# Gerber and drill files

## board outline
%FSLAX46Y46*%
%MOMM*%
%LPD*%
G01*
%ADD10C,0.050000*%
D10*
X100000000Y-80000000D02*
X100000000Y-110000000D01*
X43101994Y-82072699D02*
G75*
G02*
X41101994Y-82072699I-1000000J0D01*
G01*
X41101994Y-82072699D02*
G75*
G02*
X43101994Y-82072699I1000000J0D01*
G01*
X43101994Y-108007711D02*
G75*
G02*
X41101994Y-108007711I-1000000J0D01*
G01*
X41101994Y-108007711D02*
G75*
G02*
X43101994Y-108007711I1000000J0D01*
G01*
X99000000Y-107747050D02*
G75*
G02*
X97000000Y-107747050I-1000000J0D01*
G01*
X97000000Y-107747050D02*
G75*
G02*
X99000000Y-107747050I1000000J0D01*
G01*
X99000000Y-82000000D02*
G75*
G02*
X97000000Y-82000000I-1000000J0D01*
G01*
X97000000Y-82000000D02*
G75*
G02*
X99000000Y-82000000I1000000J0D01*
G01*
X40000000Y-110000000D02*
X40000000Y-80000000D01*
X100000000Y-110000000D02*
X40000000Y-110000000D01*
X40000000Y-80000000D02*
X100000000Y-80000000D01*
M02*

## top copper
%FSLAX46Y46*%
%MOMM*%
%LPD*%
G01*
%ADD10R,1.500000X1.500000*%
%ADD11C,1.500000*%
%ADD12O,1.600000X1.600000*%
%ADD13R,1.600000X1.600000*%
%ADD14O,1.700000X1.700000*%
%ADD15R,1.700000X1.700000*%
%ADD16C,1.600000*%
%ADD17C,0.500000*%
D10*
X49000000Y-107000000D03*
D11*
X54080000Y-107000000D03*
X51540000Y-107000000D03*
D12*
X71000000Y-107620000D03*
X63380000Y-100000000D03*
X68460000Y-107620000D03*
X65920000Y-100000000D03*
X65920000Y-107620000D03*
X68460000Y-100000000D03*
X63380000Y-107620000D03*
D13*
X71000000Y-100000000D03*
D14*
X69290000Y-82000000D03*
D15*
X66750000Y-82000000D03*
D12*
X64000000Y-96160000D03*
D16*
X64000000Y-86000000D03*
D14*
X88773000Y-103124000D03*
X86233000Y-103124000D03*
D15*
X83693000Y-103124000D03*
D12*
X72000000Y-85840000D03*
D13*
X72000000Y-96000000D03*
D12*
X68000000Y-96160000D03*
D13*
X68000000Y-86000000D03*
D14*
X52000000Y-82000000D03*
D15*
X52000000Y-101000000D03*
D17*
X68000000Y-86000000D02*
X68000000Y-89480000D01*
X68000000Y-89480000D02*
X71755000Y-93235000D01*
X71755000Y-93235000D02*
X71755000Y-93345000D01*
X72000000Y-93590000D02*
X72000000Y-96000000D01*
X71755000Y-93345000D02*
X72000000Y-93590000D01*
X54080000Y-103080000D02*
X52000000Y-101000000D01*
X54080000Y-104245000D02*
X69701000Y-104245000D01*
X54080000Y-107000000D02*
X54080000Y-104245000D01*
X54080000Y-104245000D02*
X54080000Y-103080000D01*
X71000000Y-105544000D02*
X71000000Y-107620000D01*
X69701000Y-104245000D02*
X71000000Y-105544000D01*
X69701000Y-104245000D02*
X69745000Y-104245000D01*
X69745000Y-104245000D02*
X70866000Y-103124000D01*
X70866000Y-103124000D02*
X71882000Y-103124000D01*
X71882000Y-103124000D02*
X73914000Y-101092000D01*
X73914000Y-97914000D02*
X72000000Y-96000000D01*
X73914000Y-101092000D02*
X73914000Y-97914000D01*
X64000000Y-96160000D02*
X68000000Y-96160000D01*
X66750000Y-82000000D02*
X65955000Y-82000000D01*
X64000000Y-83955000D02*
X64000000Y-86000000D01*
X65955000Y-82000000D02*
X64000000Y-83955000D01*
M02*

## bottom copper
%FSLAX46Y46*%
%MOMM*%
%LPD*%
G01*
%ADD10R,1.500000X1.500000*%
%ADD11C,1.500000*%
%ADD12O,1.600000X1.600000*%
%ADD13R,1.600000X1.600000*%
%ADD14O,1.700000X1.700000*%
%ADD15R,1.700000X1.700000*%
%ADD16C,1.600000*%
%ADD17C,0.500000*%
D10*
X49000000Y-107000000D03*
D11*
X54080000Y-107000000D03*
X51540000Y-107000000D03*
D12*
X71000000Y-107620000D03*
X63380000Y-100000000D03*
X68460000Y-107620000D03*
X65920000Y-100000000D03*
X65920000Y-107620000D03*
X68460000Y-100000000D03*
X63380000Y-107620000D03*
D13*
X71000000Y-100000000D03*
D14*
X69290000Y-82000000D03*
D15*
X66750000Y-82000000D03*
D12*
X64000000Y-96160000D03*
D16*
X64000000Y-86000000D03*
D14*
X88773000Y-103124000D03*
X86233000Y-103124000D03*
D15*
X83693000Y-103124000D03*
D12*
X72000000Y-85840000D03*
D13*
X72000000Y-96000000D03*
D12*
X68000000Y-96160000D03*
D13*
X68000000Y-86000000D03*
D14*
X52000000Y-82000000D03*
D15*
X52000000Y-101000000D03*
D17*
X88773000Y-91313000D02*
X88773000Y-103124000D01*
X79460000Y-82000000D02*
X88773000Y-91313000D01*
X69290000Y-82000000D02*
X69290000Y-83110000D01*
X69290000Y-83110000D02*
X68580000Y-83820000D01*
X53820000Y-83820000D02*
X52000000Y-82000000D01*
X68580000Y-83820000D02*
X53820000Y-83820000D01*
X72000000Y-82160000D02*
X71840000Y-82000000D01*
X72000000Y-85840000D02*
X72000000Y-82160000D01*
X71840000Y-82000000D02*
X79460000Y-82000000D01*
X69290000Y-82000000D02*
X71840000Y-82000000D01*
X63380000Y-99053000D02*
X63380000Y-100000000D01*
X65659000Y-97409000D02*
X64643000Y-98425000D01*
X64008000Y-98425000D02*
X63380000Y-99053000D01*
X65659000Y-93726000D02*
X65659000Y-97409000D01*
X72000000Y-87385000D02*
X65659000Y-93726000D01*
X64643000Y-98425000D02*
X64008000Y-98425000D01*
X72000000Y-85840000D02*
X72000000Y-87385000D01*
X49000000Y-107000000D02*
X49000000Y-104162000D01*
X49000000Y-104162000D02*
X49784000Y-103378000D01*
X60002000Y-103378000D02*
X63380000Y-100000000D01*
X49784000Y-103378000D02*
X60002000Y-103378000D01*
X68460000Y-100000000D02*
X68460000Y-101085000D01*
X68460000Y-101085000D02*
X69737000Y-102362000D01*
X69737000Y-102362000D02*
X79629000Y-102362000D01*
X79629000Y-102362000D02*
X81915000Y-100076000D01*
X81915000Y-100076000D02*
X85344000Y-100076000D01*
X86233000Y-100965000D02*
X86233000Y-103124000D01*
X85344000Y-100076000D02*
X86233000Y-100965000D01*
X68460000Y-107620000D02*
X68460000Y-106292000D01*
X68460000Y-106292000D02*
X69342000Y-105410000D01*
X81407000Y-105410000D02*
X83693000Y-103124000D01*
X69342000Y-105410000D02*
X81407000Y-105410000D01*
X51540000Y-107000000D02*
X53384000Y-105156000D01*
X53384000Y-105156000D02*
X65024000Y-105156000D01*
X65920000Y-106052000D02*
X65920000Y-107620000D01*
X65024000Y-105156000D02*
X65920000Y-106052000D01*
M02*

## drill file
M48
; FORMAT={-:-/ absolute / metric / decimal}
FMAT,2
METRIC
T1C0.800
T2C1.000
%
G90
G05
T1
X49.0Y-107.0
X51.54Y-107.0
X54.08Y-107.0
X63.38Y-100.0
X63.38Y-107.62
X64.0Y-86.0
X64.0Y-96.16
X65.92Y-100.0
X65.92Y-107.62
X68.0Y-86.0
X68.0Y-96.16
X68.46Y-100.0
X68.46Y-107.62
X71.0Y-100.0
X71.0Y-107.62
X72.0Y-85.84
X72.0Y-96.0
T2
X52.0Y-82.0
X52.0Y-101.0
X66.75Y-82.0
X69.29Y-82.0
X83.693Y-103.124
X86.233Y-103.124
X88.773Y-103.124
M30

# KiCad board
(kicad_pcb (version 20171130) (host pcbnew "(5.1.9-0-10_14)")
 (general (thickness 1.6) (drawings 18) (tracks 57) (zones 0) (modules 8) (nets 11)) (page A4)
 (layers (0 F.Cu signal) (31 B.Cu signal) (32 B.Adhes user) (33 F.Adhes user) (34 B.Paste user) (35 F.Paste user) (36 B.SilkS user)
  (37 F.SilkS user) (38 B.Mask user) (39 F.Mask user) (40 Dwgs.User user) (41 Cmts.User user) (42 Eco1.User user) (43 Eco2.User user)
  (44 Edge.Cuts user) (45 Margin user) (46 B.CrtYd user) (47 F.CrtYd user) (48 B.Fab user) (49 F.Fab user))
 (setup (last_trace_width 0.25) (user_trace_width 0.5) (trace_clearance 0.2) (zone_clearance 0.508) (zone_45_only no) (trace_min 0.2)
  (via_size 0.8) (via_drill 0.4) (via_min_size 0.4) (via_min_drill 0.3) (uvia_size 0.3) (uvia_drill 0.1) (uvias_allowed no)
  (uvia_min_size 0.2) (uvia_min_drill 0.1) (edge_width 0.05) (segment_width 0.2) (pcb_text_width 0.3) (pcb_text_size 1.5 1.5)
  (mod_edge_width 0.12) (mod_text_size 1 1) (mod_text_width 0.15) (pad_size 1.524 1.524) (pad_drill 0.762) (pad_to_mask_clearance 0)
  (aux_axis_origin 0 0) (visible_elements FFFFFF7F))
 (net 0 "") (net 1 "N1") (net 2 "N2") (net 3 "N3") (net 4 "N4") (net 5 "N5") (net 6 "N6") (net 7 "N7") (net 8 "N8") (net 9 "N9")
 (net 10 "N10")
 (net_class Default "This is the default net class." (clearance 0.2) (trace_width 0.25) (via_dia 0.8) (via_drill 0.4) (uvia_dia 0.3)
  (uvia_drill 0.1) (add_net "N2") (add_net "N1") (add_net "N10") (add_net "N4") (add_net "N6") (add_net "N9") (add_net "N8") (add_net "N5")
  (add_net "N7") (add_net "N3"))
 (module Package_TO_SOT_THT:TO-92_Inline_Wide (layer F.Cu) (at 49 107)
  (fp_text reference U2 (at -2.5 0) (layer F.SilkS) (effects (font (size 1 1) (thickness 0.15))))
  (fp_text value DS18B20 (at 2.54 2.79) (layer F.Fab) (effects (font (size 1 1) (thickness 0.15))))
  (pad 1 thru_hole rect (at 0 0) (size 1.5 1.5) (drill 0.8) (layers *.Cu *.Mask) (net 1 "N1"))
  (pad 3 thru_hole circle (at 5.08 0) (size 1.5 1.5) (drill 0.8) (layers *.Cu *.Mask) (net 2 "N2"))
  (pad 2 thru_hole circle (at 2.54 0) (size 1.5 1.5) (drill 0.8) (layers *.Cu *.Mask) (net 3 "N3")))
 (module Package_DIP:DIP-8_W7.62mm (layer F.Cu) (at 71 100 270)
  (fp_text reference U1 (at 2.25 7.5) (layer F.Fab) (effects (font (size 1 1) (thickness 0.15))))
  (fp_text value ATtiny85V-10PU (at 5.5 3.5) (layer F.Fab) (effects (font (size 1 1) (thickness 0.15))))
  (pad 8 thru_hole oval (at 7.62 0 270) (size 1.6 1.6) (drill 0.8) (layers *.Cu *.Mask) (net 2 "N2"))
  (pad 4 thru_hole oval (at 0 7.62 270) (size 1.6 1.6) (drill 0.8) (layers *.Cu *.Mask) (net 1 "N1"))
  (pad 7 thru_hole oval (at 7.62 2.54 270) (size 1.6 1.6) (drill 0.8) (layers *.Cu *.Mask) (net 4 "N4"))
  (pad 3 thru_hole oval (at 0 5.08 270) (size 1.6 1.6) (drill 0.8) (layers *.Cu *.Mask) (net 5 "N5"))
  (pad 6 thru_hole oval (at 7.62 5.08 270) (size 1.6 1.6) (drill 0.8) (layers *.Cu *.Mask) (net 3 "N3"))
  (pad 2 thru_hole oval (at 0 2.54 270) (size 1.6 1.6) (drill 0.8) (layers *.Cu *.Mask) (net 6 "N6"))
  (pad 5 thru_hole oval (at 7.62 7.62 270) (size 1.6 1.6) (drill 0.8) (layers *.Cu *.Mask) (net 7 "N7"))
  (pad 1 thru_hole rect (at 0 0 270) (size 1.6 1.6) (drill 0.8) (layers *.Cu *.Mask) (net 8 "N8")))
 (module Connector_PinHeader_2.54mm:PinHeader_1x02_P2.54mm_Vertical (layer F.Cu) (at 66.75 82 90)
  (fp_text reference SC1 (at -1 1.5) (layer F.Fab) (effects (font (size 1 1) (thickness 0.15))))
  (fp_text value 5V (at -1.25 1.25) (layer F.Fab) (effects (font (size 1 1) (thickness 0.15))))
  (pad 2 thru_hole oval (at 0 2.54 90) (size 1.7 1.7) (drill 1) (layers *.Cu *.Mask) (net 1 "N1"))
  (pad 1 thru_hole rect (at 0 0 90) (size 1.7 1.7) (drill 1) (layers *.Cu *.Mask) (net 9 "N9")))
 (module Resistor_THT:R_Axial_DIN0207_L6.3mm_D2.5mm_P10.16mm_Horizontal (layer F.Cu) (at 64 86 270)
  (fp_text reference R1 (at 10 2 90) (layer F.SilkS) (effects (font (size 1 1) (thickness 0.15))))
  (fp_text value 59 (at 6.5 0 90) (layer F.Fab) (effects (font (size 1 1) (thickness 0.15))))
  (pad 2 thru_hole oval (at 10.16 0 270) (size 1.6 1.6) (drill 0.8) (layers *.Cu *.Mask) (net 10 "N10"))
  (pad 1 thru_hole circle (at 0 0 270) (size 1.6 1.6) (drill 0.8) (layers *.Cu *.Mask) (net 9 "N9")))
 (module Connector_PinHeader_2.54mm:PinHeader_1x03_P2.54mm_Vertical (layer F.Cu) (at 83.693 103.124 90)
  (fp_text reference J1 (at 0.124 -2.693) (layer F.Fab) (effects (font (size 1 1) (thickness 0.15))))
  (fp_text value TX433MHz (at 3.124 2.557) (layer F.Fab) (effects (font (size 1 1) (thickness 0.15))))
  (pad 3 thru_hole oval (at 0 5.08 90) (size 1.7 1.7) (drill 1) (layers *.Cu *.Mask) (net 1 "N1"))
  (pad 2 thru_hole oval (at 0 2.54 90) (size 1.7 1.7) (drill 1) (layers *.Cu *.Mask) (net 6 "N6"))
  (pad 1 thru_hole rect (at 0 0 90) (size 1.7 1.7) (drill 1) (layers *.Cu *.Mask) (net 4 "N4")))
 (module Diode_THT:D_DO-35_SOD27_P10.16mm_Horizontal (layer F.Cu) (at 72 96 90)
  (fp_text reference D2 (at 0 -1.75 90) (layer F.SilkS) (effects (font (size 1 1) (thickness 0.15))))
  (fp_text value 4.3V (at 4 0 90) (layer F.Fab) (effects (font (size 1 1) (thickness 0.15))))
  (pad 2 thru_hole oval (at 10.16 0 90) (size 1.6 1.6) (drill 0.8) (layers *.Cu *.Mask) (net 1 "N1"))
  (pad 1 thru_hole rect (at 0 0 90) (size 1.6 1.6) (drill 0.8) (layers *.Cu *.Mask) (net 2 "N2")))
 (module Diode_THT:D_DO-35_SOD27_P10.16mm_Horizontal (layer F.Cu) (at 68 86 270)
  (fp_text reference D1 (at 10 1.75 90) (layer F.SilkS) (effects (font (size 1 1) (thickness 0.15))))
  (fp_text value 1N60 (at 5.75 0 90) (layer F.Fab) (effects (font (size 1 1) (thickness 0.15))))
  (pad 2 thru_hole oval (at 10.16 0 270) (size 1.6 1.6) (drill 0.8) (layers *.Cu *.Mask) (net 10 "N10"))
  (pad 1 thru_hole rect (at 0 0 270) (size 1.6 1.6) (drill 0.8) (layers *.Cu *.Mask) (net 2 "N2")))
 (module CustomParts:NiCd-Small (layer F.Cu) (at 52 101 90)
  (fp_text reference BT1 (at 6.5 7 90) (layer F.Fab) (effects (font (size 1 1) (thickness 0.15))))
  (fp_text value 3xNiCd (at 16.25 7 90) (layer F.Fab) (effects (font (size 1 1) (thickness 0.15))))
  (pad 2 thru_hole oval (at 19 0 90) (size 1.7 1.7) (drill 1) (layers *.Cu *.Mask) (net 1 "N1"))
  (pad 1 thru_hole rect (at 0 0 90) (size 1.7 1.7) (drill 1) (layers *.Cu *.Mask) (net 2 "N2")))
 (gr_line (start 100 80) (end 100 110) (layer Edge.Cuts) (width 0.05))
 (gr_circle (center 42.101994 82.072699) (end 42.101994 83.072699) (layer Edge.Cuts) (width 0.05))
 (gr_circle (center 42.101994 108.007711) (end 42.101994 109.007711) (layer Edge.Cuts) (width 0.05))
 (gr_circle (center 98 107.74705) (end 98 108.74705) (layer Edge.Cuts) (width 0.05))
 (gr_circle (center 98 82) (end 98 83) (layer Edge.Cuts) (width 0.05))
 (gr_line (start 40 110) (end 40 80) (layer Edge.Cuts) (width 0.05))
 (gr_line (start 100 110) (end 40 110) (layer Edge.Cuts) (width 0.05))
 (gr_line (start 40 80) (end 100 80) (layer Edge.Cuts) (width 0.05))
 (segment (start 88.773 91.313) (end 88.773 103.124) (width 0.5) (layer B.Cu) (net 1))
 (segment (start 79.46 82) (end 88.773 91.313) (width 0.5) (layer B.Cu) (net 1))
 (segment (start 69.29 82) (end 69.29 83.11) (width 0.5) (layer B.Cu) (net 1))
 (segment (start 69.29 83.11) (end 68.58 83.82) (width 0.5) (layer B.Cu) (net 1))
 (segment (start 53.82 83.82) (end 52 82) (width 0.5) (layer B.Cu) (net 1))
 (segment (start 68.58 83.82) (end 53.82 83.82) (width 0.5) (layer B.Cu) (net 1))
 (segment (start 72 82.16) (end 71.84 82) (width 0.5) (layer B.Cu) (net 1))
 (segment (start 72 85.84) (end 72 82.16) (width 0.5) (layer B.Cu) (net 1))
 (segment (start 71.84 82) (end 79.46 82) (width 0.5) (layer B.Cu) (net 1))
 (segment (start 69.29 82) (end 71.84 82) (width 0.5) (layer B.Cu) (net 1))
 (segment (start 63.38 99.053) (end 63.38 100) (width 0.5) (layer B.Cu) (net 1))
 (segment (start 65.659 97.409) (end 64.643 98.425) (width 0.5) (layer B.Cu) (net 1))
 (segment (start 64.008 98.425) (end 63.38 99.053) (width 0.5) (layer B.Cu) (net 1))
 (segment (start 65.659 93.726) (end 65.659 97.409) (width 0.5) (layer B.Cu) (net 1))
 (segment (start 72 87.385) (end 65.659 93.726) (width 0.5) (layer B.Cu) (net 1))
 (segment (start 64.643 98.425) (end 64.008 98.425) (width 0.5) (layer B.Cu) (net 1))
 (segment (start 72 85.84) (end 72 87.385) (width 0.5) (layer B.Cu) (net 1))
 (segment (start 49 107) (end 49 104.162) (width 0.5) (layer B.Cu) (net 1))
 (segment (start 49 104.162) (end 49.784 103.378) (width 0.5) (layer B.Cu) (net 1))
 (segment (start 60.002 103.378) (end 63.38 100) (width 0.5) (layer B.Cu) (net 1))
 (segment (start 49.784 103.378) (end 60.002 103.378) (width 0.5) (layer B.Cu) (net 1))
 (segment (start 68 86) (end 68 89.48) (width 0.5) (layer F.Cu) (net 2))
 (segment (start 68 89.48) (end 71.755 93.235) (width 0.5) (layer F.Cu) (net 2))
 (segment (start 71.755 93.235) (end 71.755 93.345) (width 0.5) (layer F.Cu) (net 2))
 (segment (start 72 93.59) (end 72 96) (width 0.5) (layer F.Cu) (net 2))
 (segment (start 71.755 93.345) (end 72 93.59) (width 0.5) (layer F.Cu) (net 2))
 (segment (start 54.08 103.08) (end 52 101) (width 0.5) (layer F.Cu) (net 2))
 (segment (start 54.08 104.245) (end 69.701 104.245) (width 0.5) (layer F.Cu) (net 2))
 (segment (start 54.08 107) (end 54.08 104.245) (width 0.5) (layer F.Cu) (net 2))
 (segment (start 54.08 104.245) (end 54.08 103.08) (width 0.5) (layer F.Cu) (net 2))
 (segment (start 71 105.544) (end 71 107.62) (width 0.5) (layer F.Cu) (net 2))
 (segment (start 69.701 104.245) (end 71 105.544) (width 0.5) (layer F.Cu) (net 2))
 (segment (start 69.701 104.245) (end 69.745 104.245) (width 0.5) (layer F.Cu) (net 2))
 (segment (start 69.745 104.245) (end 70.866 103.124) (width 0.5) (layer F.Cu) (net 2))
 (segment (start 70.866 103.124) (end 71.882 103.124) (width 0.5) (layer F.Cu) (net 2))
 (segment (start 71.882 103.124) (end 73.914 101.092) (width 0.5) (layer F.Cu) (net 2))
 (segment (start 73.914 97.914) (end 72 96) (width 0.5) (layer F.Cu) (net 2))
 (segment (start 73.914 101.092) (end 73.914 97.914) (width 0.5) (layer F.Cu) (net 2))
 (segment (start 64 96.16) (end 68 96.16) (width 0.5) (layer F.Cu) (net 10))
 (segment (start 68.46 100) (end 68.46 101.085) (width 0.5) (layer B.Cu) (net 6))
 (segment (start 68.46 101.085) (end 69.737 102.362) (width 0.5) (layer B.Cu) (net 6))
 (segment (start 69.737 102.362) (end 79.629 102.362) (width 0.5) (layer B.Cu) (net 6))
 (segment (start 79.629 102.362) (end 81.915 100.076) (width 0.5) (layer B.Cu) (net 6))
 (segment (start 81.915 100.076) (end 85.344 100.076) (width 0.5) (layer B.Cu) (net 6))
 (segment (start 86.233 100.965) (end 86.233 103.124) (width 0.5) (layer B.Cu) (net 6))
 (segment (start 85.344 100.076) (end 86.233 100.965) (width 0.5) (layer B.Cu) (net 6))
 (segment (start 68.46 107.62) (end 68.46 106.292) (width 0.5) (layer B.Cu) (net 4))
 (segment (start 68.46 106.292) (end 69.342 105.41) (width 0.5) (layer B.Cu) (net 4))
 (segment (start 81.407 105.41) (end 83.693 103.124) (width 0.5) (layer B.Cu) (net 4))
 (segment (start 69.342 105.41) (end 81.407 105.41) (width 0.5) (layer B.Cu) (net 4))
 (segment (start 66.75 82) (end 65.955 82) (width 0.5) (layer F.Cu) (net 9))
 (segment (start 64 83.955) (end 64 86) (width 0.5) (layer F.Cu) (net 9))
 (segment (start 65.955 82) (end 64 83.955) (width 0.5) (layer F.Cu) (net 9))
 (segment (start 51.54 107) (end 53.384 105.156) (width 0.5) (layer B.Cu) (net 3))
 (segment (start 53.384 105.156) (end 65.024 105.156) (width 0.5) (layer B.Cu) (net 3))
 (segment (start 65.92 106.052) (end 65.92 107.62) (width 0.5) (layer B.Cu) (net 3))
 (segment (start 65.024 105.156) (end 65.92 106.052) (width 0.5) (layer B.Cu) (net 3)))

